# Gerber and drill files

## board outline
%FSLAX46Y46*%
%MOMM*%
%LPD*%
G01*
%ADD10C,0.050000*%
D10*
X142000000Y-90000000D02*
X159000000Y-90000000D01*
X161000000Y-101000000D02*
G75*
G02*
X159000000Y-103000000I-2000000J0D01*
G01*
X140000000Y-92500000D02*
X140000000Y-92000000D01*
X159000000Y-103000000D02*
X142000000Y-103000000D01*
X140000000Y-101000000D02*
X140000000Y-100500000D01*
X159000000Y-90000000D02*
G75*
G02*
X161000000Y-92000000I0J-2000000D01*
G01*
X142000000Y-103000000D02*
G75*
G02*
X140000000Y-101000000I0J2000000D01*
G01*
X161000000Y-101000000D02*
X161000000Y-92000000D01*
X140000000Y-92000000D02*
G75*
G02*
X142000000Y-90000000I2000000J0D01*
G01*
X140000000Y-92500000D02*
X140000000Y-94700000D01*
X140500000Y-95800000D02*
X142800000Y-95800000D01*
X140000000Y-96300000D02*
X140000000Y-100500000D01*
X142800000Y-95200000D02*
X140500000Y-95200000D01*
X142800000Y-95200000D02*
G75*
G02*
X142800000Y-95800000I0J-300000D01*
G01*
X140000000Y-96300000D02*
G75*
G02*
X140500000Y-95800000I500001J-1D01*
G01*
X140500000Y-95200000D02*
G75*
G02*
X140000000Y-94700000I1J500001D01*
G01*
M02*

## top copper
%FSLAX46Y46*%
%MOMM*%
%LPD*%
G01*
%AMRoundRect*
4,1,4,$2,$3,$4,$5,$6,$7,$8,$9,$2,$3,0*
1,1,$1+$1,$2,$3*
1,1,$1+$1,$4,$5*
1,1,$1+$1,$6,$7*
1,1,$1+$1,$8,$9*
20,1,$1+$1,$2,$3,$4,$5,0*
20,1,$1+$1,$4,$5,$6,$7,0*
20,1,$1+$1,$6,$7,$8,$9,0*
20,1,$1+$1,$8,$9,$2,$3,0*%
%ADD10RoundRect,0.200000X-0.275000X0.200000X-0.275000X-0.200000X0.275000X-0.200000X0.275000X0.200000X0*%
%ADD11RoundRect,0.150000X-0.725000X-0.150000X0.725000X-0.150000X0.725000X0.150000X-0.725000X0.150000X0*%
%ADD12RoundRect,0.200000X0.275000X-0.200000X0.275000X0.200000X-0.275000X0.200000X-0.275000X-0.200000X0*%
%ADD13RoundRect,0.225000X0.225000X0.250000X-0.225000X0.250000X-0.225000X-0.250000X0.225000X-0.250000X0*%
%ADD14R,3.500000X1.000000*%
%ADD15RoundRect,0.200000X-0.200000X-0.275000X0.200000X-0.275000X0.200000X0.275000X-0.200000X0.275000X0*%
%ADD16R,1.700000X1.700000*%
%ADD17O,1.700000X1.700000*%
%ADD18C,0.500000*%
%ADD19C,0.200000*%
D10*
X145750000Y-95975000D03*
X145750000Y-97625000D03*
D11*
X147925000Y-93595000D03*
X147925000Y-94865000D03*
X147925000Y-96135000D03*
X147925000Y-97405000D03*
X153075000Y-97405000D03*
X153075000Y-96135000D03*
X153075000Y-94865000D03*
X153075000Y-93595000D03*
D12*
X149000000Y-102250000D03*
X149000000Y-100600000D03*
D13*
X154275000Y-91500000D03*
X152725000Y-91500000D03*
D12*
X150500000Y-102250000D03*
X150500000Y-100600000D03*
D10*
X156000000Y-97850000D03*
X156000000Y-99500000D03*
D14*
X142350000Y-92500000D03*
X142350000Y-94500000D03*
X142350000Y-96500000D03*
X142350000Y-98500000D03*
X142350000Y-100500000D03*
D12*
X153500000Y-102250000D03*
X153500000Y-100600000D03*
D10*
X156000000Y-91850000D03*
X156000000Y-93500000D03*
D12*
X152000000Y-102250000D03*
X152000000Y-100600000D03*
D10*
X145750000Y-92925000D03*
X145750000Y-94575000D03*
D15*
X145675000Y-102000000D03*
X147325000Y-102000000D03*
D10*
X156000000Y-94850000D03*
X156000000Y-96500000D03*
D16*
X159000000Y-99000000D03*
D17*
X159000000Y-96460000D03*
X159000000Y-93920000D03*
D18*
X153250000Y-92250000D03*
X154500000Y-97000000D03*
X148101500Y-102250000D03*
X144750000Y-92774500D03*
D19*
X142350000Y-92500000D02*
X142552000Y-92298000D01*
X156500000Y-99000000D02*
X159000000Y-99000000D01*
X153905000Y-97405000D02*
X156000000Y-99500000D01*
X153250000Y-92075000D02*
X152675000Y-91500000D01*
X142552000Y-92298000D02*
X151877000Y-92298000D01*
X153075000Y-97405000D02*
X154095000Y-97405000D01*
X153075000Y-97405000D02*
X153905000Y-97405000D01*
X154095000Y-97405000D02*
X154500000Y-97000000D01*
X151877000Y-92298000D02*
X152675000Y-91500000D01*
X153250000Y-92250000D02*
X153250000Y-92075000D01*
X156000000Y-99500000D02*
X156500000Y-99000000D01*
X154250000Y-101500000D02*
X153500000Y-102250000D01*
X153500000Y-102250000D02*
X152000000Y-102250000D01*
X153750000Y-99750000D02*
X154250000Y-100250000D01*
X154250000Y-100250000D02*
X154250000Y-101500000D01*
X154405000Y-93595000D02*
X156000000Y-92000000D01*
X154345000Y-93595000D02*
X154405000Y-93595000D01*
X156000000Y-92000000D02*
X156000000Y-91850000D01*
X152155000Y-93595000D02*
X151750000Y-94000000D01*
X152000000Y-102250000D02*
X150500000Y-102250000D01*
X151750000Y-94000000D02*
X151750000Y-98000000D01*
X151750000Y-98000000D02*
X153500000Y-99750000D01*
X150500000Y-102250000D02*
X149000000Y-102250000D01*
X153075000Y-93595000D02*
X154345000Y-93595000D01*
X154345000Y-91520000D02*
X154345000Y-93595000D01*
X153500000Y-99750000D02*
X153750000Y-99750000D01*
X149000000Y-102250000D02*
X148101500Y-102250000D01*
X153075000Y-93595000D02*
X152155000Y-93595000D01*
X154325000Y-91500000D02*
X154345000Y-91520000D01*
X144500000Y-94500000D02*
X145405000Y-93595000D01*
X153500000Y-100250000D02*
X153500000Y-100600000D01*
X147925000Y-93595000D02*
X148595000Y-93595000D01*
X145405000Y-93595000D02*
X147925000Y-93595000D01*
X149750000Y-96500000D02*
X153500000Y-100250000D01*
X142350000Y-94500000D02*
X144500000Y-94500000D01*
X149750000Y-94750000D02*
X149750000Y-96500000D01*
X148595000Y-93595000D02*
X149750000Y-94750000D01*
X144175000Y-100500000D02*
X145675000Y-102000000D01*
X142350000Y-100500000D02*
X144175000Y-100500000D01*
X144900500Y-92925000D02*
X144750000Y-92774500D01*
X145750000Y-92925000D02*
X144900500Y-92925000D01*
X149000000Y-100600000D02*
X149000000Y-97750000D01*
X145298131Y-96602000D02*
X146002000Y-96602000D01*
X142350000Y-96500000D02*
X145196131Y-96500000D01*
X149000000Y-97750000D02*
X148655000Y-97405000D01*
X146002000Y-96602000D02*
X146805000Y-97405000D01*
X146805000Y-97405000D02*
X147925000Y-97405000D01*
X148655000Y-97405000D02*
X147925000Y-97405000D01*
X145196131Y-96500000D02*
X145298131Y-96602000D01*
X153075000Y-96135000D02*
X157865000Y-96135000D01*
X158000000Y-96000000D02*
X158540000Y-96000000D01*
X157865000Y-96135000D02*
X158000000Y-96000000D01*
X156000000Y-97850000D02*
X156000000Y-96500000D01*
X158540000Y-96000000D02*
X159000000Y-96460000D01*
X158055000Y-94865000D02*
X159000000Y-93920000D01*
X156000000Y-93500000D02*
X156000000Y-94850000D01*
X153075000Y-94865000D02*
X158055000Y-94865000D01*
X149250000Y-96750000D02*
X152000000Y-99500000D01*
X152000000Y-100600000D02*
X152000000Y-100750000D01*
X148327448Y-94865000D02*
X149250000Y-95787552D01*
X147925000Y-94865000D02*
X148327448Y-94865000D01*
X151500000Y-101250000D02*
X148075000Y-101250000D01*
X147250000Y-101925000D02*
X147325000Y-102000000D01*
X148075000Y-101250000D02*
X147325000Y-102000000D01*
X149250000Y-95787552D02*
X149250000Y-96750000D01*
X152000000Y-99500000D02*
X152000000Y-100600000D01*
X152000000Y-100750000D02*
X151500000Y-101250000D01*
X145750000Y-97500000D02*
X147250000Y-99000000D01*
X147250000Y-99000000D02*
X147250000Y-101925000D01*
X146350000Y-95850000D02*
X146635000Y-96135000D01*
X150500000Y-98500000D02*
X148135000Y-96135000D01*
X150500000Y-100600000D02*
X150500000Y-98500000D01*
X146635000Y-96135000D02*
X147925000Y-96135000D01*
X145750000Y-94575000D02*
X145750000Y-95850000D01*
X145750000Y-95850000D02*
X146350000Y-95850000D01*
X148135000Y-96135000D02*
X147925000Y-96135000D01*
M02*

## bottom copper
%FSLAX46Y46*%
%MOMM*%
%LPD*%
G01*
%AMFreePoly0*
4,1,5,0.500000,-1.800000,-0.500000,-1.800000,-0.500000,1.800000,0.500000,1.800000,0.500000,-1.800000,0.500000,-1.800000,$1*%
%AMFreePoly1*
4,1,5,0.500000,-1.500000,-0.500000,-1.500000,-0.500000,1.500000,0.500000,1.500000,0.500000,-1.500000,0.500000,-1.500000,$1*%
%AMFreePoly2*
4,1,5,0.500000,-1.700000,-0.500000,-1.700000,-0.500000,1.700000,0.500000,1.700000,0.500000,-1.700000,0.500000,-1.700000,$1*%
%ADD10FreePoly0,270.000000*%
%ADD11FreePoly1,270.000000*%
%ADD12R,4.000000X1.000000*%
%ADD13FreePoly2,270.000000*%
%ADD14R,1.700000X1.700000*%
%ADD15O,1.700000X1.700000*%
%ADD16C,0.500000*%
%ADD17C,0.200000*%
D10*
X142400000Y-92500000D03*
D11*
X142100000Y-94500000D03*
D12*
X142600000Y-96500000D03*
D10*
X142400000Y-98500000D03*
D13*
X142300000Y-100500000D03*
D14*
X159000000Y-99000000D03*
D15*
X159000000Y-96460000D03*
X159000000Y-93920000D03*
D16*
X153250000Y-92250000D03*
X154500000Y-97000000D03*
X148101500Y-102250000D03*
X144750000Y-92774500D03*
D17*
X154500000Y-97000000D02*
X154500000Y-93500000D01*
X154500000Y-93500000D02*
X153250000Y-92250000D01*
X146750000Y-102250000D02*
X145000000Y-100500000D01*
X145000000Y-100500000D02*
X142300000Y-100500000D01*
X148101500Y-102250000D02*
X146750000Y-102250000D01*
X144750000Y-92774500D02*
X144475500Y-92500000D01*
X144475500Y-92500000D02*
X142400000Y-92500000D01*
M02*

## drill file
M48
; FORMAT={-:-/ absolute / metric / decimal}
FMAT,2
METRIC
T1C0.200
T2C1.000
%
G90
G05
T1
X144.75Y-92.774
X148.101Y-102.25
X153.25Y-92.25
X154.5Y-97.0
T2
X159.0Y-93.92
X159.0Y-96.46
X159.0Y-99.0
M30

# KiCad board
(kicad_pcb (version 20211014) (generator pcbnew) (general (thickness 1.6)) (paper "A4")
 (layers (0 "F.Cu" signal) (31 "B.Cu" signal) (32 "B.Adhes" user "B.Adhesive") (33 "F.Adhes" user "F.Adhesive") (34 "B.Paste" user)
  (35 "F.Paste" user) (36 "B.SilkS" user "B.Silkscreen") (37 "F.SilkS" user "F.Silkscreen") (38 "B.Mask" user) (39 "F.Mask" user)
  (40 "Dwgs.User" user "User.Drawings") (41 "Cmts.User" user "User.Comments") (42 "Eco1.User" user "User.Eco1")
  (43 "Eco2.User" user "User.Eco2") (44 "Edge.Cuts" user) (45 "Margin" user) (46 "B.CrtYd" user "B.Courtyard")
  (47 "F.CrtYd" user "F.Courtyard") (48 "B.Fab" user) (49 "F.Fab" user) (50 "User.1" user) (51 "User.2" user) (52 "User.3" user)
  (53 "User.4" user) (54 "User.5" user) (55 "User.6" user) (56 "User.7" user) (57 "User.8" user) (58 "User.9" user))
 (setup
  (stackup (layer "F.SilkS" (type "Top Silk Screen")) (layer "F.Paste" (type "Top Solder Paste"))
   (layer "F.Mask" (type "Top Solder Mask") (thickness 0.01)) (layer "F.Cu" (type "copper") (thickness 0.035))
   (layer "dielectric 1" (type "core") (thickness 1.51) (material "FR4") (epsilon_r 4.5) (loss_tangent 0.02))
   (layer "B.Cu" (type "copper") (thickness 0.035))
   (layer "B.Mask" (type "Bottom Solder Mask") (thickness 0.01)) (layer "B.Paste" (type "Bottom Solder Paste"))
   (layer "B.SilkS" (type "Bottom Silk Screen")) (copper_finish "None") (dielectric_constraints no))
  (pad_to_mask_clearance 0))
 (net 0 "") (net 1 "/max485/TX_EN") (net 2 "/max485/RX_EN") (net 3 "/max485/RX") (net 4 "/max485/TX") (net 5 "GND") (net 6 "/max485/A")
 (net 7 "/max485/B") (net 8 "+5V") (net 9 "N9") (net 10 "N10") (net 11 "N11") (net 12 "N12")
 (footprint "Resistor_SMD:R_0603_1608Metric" (layer "F.Cu") (at 145.75 96.8 -90)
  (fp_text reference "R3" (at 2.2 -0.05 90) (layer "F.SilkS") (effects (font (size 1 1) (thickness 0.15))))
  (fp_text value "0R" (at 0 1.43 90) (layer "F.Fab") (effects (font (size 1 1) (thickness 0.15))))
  (pad "1" smd roundrect (at -0.825 0 270) (size 0.8 0.95) (layers "F.Cu" "F.Paste" "F.Mask") (roundrect_rratio 0.25)
   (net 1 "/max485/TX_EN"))
  (pad "2" smd roundrect (at 0.825 0 270) (size 0.8 0.95) (layers "F.Cu" "F.Paste" "F.Mask") (roundrect_rratio 0.25) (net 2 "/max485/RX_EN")))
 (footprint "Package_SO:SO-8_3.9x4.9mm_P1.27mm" (layer "F.Cu") (at 150.5 95.5)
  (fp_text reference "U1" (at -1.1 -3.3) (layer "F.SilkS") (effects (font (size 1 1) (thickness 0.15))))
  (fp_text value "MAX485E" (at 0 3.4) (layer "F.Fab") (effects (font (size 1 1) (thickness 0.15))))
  (pad "1" smd roundrect (at -2.575 -1.905) (size 1.75 0.6) (layers "F.Cu" "F.Paste" "F.Mask") (roundrect_rratio 0.25) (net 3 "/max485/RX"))
  (pad "2" smd roundrect (at -2.575 -0.635) (size 1.75 0.6) (layers "F.Cu" "F.Paste" "F.Mask") (roundrect_rratio 0.25)
   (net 2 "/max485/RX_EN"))
  (pad "3" smd roundrect (at -2.575 0.635) (size 1.75 0.6) (layers "F.Cu" "F.Paste" "F.Mask") (roundrect_rratio 0.25)
   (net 1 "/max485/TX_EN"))
  (pad "4" smd roundrect (at -2.575 1.905) (size 1.75 0.6) (layers "F.Cu" "F.Paste" "F.Mask") (roundrect_rratio 0.25) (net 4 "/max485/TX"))
  (pad "5" smd roundrect (at 2.575 1.905) (size 1.75 0.6) (layers "F.Cu" "F.Paste" "F.Mask") (roundrect_rratio 0.25) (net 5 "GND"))
  (pad "6" smd roundrect (at 2.575 0.635) (size 1.75 0.6) (layers "F.Cu" "F.Paste" "F.Mask") (roundrect_rratio 0.25) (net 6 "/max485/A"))
  (pad "7" smd roundrect (at 2.575 -0.635) (size 1.75 0.6) (layers "F.Cu" "F.Paste" "F.Mask") (roundrect_rratio 0.25) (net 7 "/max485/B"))
  (pad "8" smd roundrect (at 2.575 -1.905) (size 1.75 0.6) (layers "F.Cu" "F.Paste" "F.Mask") (roundrect_rratio 0.25) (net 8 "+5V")))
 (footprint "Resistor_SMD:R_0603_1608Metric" (layer "F.Cu") (at 149 101.425 90)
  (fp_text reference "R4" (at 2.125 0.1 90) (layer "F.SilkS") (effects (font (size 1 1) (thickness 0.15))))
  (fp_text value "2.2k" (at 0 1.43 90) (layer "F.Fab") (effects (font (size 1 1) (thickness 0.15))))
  (pad "1" smd roundrect (at -0.825 0 90) (size 0.8 0.95) (layers "F.Cu" "F.Paste" "F.Mask") (roundrect_rratio 0.25) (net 8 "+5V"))
  (pad "2" smd roundrect (at 0.825 0 90) (size 0.8 0.95) (layers "F.Cu" "F.Paste" "F.Mask") (roundrect_rratio 0.25) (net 4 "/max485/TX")))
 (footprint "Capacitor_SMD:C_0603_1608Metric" (layer "F.Cu") (at 153.5 91.5 180)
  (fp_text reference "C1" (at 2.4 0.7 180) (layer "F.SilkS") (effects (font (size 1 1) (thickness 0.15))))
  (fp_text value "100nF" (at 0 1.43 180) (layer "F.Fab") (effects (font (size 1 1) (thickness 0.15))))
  (pad "1" smd roundrect (at -0.775 0 180) (size 0.9 0.95) (layers "F.Cu" "F.Paste" "F.Mask") (roundrect_rratio 0.25) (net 8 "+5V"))
  (pad "2" smd roundrect (at 0.775 0 180) (size 0.9 0.95) (layers "F.Cu" "F.Paste" "F.Mask") (roundrect_rratio 0.25) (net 5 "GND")))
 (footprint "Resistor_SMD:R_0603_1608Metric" (layer "F.Cu") (at 150.5 101.425 90)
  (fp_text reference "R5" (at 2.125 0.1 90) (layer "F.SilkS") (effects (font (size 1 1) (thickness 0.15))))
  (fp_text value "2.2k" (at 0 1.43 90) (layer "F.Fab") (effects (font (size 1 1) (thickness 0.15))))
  (pad "1" smd roundrect (at -0.825 0 90) (size 0.8 0.95) (layers "F.Cu" "F.Paste" "F.Mask") (roundrect_rratio 0.25) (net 8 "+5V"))
  (pad "2" smd roundrect (at 0.825 0 90) (size 0.8 0.95) (layers "F.Cu" "F.Paste" "F.Mask") (roundrect_rratio 0.25) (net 1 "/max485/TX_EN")))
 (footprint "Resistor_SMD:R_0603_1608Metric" (layer "F.Cu") (at 156 98.675 -90)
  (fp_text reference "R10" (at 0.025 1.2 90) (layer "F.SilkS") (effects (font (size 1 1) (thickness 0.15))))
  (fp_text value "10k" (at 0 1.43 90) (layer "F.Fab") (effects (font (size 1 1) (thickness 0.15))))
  (pad "1" smd roundrect (at -0.825 0 270) (size 0.8 0.95) (layers "F.Cu" "F.Paste" "F.Mask") (roundrect_rratio 0.25) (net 6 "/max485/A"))
  (pad "2" smd roundrect (at 0.825 0 270) (size 0.8 0.95) (layers "F.Cu" "F.Paste" "F.Mask") (roundrect_rratio 0.25) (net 5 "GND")))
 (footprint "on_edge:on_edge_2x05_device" (layer "F.Cu") (at 140 96.5 -90)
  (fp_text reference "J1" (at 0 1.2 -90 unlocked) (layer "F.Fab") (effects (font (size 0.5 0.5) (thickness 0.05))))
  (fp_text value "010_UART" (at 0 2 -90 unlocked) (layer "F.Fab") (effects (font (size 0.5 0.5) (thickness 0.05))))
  (fp_line (start -4 0) (end -1.8 0) (layer "Edge.Cuts") (width 0.05))
  (fp_line (start -0.7 -0.5) (end -0.7 -2.8) (layer "Edge.Cuts") (width 0.05))
  (fp_line (start -0.2 0) (end 4 0) (layer "Edge.Cuts") (width 0.05))
  (fp_line (start -1.3 -2.8) (end -1.3 -0.5) (layer "Edge.Cuts") (width 0.05))
  (fp_arc (start -1.3 -2.8) (mid -1 -3.1) (end -0.7 -2.8) (layer "Edge.Cuts") (width 0.05))
  (fp_arc (start -0.2 0) (mid -0.553553 -0.146447) (end -0.7 -0.5) (layer "Edge.Cuts") (width 0.05))
  (fp_arc (start -1.3 -0.5) (mid -1.446447 -0.146447) (end -1.8 0) (layer "Edge.Cuts") (width 0.05))
  (pad "1" smd rect (at -4 -2.35 90) (size 1 3.5) (layers "F.Cu" "F.Mask") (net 5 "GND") (zone_connect 0))
  (pad "2" smd rect (at -2 -2.35 270) (size 1 3.5) (layers "F.Cu" "F.Mask") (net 3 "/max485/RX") (zone_connect 0))
  (pad "3" smd rect (at 0 -2.35 270) (size 1 3.5) (layers "F.Cu" "F.Mask") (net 4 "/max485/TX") (zone_connect 0))
  (pad "4" smd rect (at 2 -2.35 90) (size 1 3.5) (layers "F.Cu" "F.Mask") (zone_connect 0))
  (pad "5" smd rect (at 4 -2.35 90) (size 1 3.5) (layers "F.Cu" "F.Mask") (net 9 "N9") (zone_connect 0))
  (pad "6" smd custom (at -4 -2.4 270) (size 1 3.6) (layers "B.Cu" "B.Mask") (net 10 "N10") (zone_connect 0)
   (options (clearance outline) (anchor rect)) (primitives))
  (pad "7" smd custom (at -2 -2.1 270) (size 1 3) (layers "B.Cu" "B.Mask") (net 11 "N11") (zone_connect 0)
   (options (clearance outline) (anchor rect)) (primitives))
  (pad "8" smd rect (at 0 -2.6 270) (size 1 4) (layers "B.Cu" "B.Mask") (zone_connect 0))
  (pad "9" smd custom (at 2 -2.4 270) (size 1 3.6) (layers "B.Cu" "B.Mask") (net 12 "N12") (zone_connect 0)
   (options (clearance outline) (anchor rect)) (primitives))
  (pad "10" smd custom (at 4 -2.3 270) (size 1 3.4) (layers "B.Cu" "B.Mask") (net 8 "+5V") (zone_connect 0)
   (options (clearance outline) (anchor rect)) (primitives)))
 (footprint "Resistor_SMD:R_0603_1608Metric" (layer "F.Cu") (at 153.5 101.425 90)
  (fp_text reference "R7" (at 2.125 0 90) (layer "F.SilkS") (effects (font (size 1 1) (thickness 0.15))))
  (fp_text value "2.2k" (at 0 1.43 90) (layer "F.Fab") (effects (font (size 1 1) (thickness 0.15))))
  (pad "1" smd roundrect (at -0.825 0 90) (size 0.8 0.95) (layers "F.Cu" "F.Paste" "F.Mask") (roundrect_rratio 0.25) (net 8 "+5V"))
  (pad "2" smd roundrect (at 0.825 0 90) (size 0.8 0.95) (layers "F.Cu" "F.Paste" "F.Mask") (roundrect_rratio 0.25) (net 3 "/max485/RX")))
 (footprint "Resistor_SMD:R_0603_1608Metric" (layer "F.Cu") (at 156 92.675 -90)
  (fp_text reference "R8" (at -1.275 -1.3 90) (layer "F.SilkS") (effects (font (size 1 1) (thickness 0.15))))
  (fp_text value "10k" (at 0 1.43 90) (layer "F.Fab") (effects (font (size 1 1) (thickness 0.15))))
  (pad "1" smd roundrect (at -0.825 0 270) (size 0.8 0.95) (layers "F.Cu" "F.Paste" "F.Mask") (roundrect_rratio 0.25) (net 8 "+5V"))
  (pad "2" smd roundrect (at 0.825 0 270) (size 0.8 0.95) (layers "F.Cu" "F.Paste" "F.Mask") (roundrect_rratio 0.25) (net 7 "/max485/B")))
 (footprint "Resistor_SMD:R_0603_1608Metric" (layer "F.Cu") (at 152 101.425 90)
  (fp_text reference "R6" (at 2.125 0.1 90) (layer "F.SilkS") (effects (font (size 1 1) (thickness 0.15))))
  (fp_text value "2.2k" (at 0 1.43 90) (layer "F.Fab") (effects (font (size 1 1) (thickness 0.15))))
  (pad "1" smd roundrect (at -0.825 0 90) (size 0.8 0.95) (layers "F.Cu" "F.Paste" "F.Mask") (roundrect_rratio 0.25) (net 8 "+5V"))
  (pad "2" smd roundrect (at 0.825 0 90) (size 0.8 0.95) (layers "F.Cu" "F.Paste" "F.Mask") (roundrect_rratio 0.25) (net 2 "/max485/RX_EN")))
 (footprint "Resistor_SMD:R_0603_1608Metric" (layer "F.Cu") (at 145.75 93.75 -90)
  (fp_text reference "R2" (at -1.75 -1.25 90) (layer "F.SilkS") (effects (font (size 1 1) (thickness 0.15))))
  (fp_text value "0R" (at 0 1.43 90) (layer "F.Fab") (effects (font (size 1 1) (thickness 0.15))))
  (pad "1" smd roundrect (at -0.825 0 270) (size 0.8 0.95) (layers "F.Cu" "F.Paste" "F.Mask") (roundrect_rratio 0.25) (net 10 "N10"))
  (pad "2" smd roundrect (at 0.825 0 270) (size 0.8 0.95) (layers "F.Cu" "F.Paste" "F.Mask") (roundrect_rratio 0.25) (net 1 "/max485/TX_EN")))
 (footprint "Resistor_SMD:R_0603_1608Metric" (layer "F.Cu") (at 146.5 102)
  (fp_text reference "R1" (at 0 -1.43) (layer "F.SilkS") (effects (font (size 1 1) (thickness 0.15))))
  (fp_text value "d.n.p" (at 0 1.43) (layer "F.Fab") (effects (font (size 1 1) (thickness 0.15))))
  (pad "1" smd roundrect (at -0.825 0) (size 0.8 0.95) (layers "F.Cu" "F.Paste" "F.Mask") (roundrect_rratio 0.25) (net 9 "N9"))
  (pad "2" smd roundrect (at 0.825 0) (size 0.8 0.95) (layers "F.Cu" "F.Paste" "F.Mask") (roundrect_rratio 0.25) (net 2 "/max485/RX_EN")))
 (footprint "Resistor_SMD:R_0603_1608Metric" (layer "F.Cu") (at 156 95.675 -90)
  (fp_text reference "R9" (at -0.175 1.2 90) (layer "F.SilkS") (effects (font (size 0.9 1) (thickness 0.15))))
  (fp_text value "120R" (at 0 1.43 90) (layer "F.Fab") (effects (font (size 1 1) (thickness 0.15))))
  (pad "1" smd roundrect (at -0.825 0 270) (size 0.8 0.95) (layers "F.Cu" "F.Paste" "F.Mask") (roundrect_rratio 0.25) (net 7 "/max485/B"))
  (pad "2" smd roundrect (at 0.825 0 270) (size 0.8 0.95) (layers "F.Cu" "F.Paste" "F.Mask") (roundrect_rratio 0.25) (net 6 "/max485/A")))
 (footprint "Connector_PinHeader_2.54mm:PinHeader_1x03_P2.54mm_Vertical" (layer "F.Cu") (at 159 99 180)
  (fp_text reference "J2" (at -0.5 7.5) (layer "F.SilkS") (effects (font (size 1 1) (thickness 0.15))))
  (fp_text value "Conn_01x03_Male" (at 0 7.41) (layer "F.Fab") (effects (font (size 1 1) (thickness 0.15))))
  (pad "1" thru_hole rect (at 0 0 180) (size 1.7 1.7) (drill 1) (layers *.Cu *.Mask) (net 5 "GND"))
  (pad "2" thru_hole oval (at 0 2.54 180) (size 1.7 1.7) (drill 1) (layers *.Cu *.Mask) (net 6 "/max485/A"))
  (pad "3" thru_hole oval (at 0 5.08 180) (size 1.7 1.7) (drill 1) (layers *.Cu *.Mask) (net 7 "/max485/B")))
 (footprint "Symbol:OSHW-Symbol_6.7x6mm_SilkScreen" (layer "B.Cu") (at 151 96.5 180)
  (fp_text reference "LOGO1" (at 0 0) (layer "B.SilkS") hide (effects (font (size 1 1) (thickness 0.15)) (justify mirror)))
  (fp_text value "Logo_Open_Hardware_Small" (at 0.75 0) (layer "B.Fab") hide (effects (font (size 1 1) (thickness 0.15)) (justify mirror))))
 (gr_line (start 142 90) (end 159 90) (layer "Edge.Cuts") (width 0.05))
 (gr_arc (start 161 101) (mid 160.414214 102.414214) (end 159 103) (layer "Edge.Cuts") (width 0.05))
 (gr_line (start 140 92.5) (end 140 92) (layer "Edge.Cuts") (width 0.05))
 (gr_line (start 159 103) (end 142 103) (layer "Edge.Cuts") (width 0.05))
 (gr_line (start 140 101) (end 140 100.5) (layer "Edge.Cuts") (width 0.05))
 (gr_arc (start 159 90) (mid 160.414214 90.585786) (end 161 92) (layer "Edge.Cuts") (width 0.05))
 (gr_arc (start 142 103) (mid 140.585786 102.414214) (end 140 101) (layer "Edge.Cuts") (width 0.05))
 (gr_line (start 161 101) (end 161 92) (layer "Edge.Cuts") (width 0.05))
 (gr_arc (start 140 92) (mid 140.585786 90.585786) (end 142 90) (layer "Edge.Cuts") (width 0.05))
 (segment (start 142.35 92.5) (end 142.552 92.298) (width 0.2) (layer "F.Cu") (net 5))
 (segment (start 156.5 99) (end 159 99) (width 0.2) (layer "F.Cu") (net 5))
 (segment (start 153.905 97.405) (end 156 99.5) (width 0.2) (layer "F.Cu") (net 5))
 (segment (start 153.25 92.075) (end 152.675 91.5) (width 0.2) (layer "F.Cu") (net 5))
 (segment (start 142.552 92.298) (end 151.877 92.298) (width 0.2) (layer "F.Cu") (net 5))
 (segment (start 153.075 97.405) (end 154.095 97.405) (width 0.2) (layer "F.Cu") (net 5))
 (segment (start 153.075 97.405) (end 153.905 97.405) (width 0.2) (layer "F.Cu") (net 5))
 (segment (start 154.095 97.405) (end 154.5 97) (width 0.2) (layer "F.Cu") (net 5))
 (segment (start 151.877 92.298) (end 152.675 91.5) (width 0.2) (layer "F.Cu") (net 5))
 (segment (start 153.25 92.25) (end 153.25 92.075) (width 0.2) (layer "F.Cu") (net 5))
 (segment (start 156 99.5) (end 156.5 99) (width 0.2) (layer "F.Cu") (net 5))
 (via (at 153.25 92.25) (size 0.5) (drill 0.2) (layers "F.Cu" "B.Cu") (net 5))
 (via (at 154.5 97) (size 0.5) (drill 0.2) (layers "F.Cu" "B.Cu") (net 5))
 (segment (start 154.5 97) (end 154.5 93.5) (width 0.2) (layer "B.Cu") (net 5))
 (segment (start 154.5 93.5) (end 153.25 92.25) (width 0.2) (layer "B.Cu") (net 5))
 (segment (start 154.25 101.5) (end 153.5 102.25) (width 0.2) (layer "F.Cu") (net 8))
 (segment (start 153.5 102.25) (end 152 102.25) (width 0.2) (layer "F.Cu") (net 8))
 (segment (start 153.75 99.75) (end 154.25 100.25) (width 0.2) (layer "F.Cu") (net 8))
 (segment (start 154.25 100.25) (end 154.25 101.5) (width 0.2) (layer "F.Cu") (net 8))
 (segment (start 154.405 93.595) (end 156 92) (width 0.2) (layer "F.Cu") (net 8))
 (segment (start 154.345 93.595) (end 154.405 93.595) (width 0.2) (layer "F.Cu") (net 8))
 (segment (start 156 92) (end 156 91.85) (width 0.2) (layer "F.Cu") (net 8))
 (segment (start 152.155 93.595) (end 151.75 94) (width 0.2) (layer "F.Cu") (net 8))
 (segment (start 152 102.25) (end 150.5 102.25) (width 0.2) (layer "F.Cu") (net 8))
 (segment (start 151.75 94) (end 151.75 98) (width 0.2) (layer "F.Cu") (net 8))
 (segment (start 151.75 98) (end 153.5 99.75) (width 0.2) (layer "F.Cu") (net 8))
 (segment (start 150.5 102.25) (end 149 102.25) (width 0.2) (layer "F.Cu") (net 8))
 (segment (start 153.075 93.595) (end 154.345 93.595) (width 0.2) (layer "F.Cu") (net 8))
 (segment (start 154.345 91.52) (end 154.345 93.595) (width 0.2) (layer "F.Cu") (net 8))
 (segment (start 153.5 99.75) (end 153.75 99.75) (width 0.2) (layer "F.Cu") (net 8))
 (segment (start 149 102.25) (end 148.1015 102.25) (width 0.2) (layer "F.Cu") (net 8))
 (segment (start 153.075 93.595) (end 152.155 93.595) (width 0.2) (layer "F.Cu") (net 8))
 (segment (start 154.325 91.5) (end 154.345 91.52) (width 0.2) (layer "F.Cu") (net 8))
 (via (at 148.1015 102.25) (size 0.5) (drill 0.2) (layers "F.Cu" "B.Cu") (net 8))
 (segment (start 146.75 102.25) (end 145 100.5) (width 0.2) (layer "B.Cu") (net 8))
 (segment (start 145 100.5) (end 142.3 100.5) (width 0.2) (layer "B.Cu") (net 8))
 (segment (start 148.1015 102.25) (end 146.75 102.25) (width 0.2) (layer "B.Cu") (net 8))
 (segment (start 144.5 94.5) (end 145.405 93.595) (width 0.2) (layer "F.Cu") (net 3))
 (segment (start 153.5 100.25) (end 153.5 100.6) (width 0.2) (layer "F.Cu") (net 3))
 (segment (start 147.925 93.595) (end 148.595 93.595) (width 0.2) (layer "F.Cu") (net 3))
 (segment (start 145.405 93.595) (end 147.925 93.595) (width 0.2) (layer "F.Cu") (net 3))
 (segment (start 149.75 96.5) (end 153.5 100.25) (width 0.2) (layer "F.Cu") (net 3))
 (segment (start 142.35 94.5) (end 144.5 94.5) (width 0.2) (layer "F.Cu") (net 3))
 (segment (start 149.75 94.75) (end 149.75 96.5) (width 0.2) (layer "F.Cu") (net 3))
 (segment (start 148.595 93.595) (end 149.75 94.75) (width 0.2) (layer "F.Cu") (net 3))
 (segment (start 144.175 100.5) (end 145.675 102) (width 0.2) (layer "F.Cu") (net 9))
 (segment (start 142.35 100.5) (end 144.175 100.5) (width 0.2) (layer "F.Cu") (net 9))
 (segment (start 144.9005 92.925) (end 144.75 92.7745) (width 0.2) (layer "F.Cu") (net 10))
 (segment (start 145.75 92.925) (end 144.9005 92.925) (width 0.2) (layer "F.Cu") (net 10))
 (via (at 144.75 92.7745) (size 0.5) (drill 0.2) (layers "F.Cu" "B.Cu") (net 10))
 (segment (start 144.75 92.7745) (end 144.4755 92.5) (width 0.2) (layer "B.Cu") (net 10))
 (segment (start 144.4755 92.5) (end 142.4 92.5) (width 0.2) (layer "B.Cu") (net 10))
 (segment (start 149 100.6) (end 149 97.75) (width 0.2) (layer "F.Cu") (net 4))
 (segment (start 145.298131 96.602) (end 146.002 96.602) (width 0.2) (layer "F.Cu") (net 4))
 (segment (start 142.35 96.5) (end 145.196131 96.5) (width 0.2) (layer "F.Cu") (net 4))
 (segment (start 149 97.75) (end 148.655 97.405) (width 0.2) (layer "F.Cu") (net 4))
 (segment (start 146.002 96.602) (end 146.805 97.405) (width 0.2) (layer "F.Cu") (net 4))
 (segment (start 146.805 97.405) (end 147.925 97.405) (width 0.2) (layer "F.Cu") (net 4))
 (segment (start 148.655 97.405) (end 147.925 97.405) (width 0.2) (layer "F.Cu") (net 4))
 (segment (start 145.196131 96.5) (end 145.298131 96.602) (width 0.2) (layer "F.Cu") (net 4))
 (segment (start 153.075 96.135) (end 157.865 96.135) (width 0.2) (layer "F.Cu") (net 6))
 (segment (start 158 96) (end 158.54 96) (width 0.2) (layer "F.Cu") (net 6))
 (segment (start 157.865 96.135) (end 158 96) (width 0.2) (layer "F.Cu") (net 6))
 (segment (start 156 97.85) (end 156 96.5) (width 0.2) (layer "F.Cu") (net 6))
 (segment (start 158.54 96) (end 159 96.46) (width 0.2) (layer "F.Cu") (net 6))
 (segment (start 158.055 94.865) (end 159 93.92) (width 0.2) (layer "F.Cu") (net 7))
 (segment (start 156 93.5) (end 156 94.85) (width 0.2) (layer "F.Cu") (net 7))
 (segment (start 153.075 94.865) (end 158.055 94.865) (width 0.2) (layer "F.Cu") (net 7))
 (segment (start 149.25 96.75) (end 152 99.5) (width 0.2) (layer "F.Cu") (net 2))
 (segment (start 152 100.6) (end 152 100.75) (width 0.2) (layer "F.Cu") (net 2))
 (segment (start 148.327448 94.865) (end 149.25 95.787552) (width 0.2) (layer "F.Cu") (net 2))
 (segment (start 147.925 94.865) (end 148.327448 94.865) (width 0.2) (layer "F.Cu") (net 2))
 (segment (start 151.5 101.25) (end 148.075 101.25) (width 0.2) (layer "F.Cu") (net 2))
 (segment (start 147.25 101.925) (end 147.325 102) (width 0.2) (layer "F.Cu") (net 2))
 (segment (start 148.075 101.25) (end 147.325 102) (width 0.2) (layer "F.Cu") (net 2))
 (segment (start 149.25 95.787552) (end 149.25 96.75) (width 0.2) (layer "F.Cu") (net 2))
 (segment (start 152 99.5) (end 152 100.6) (width 0.2) (layer "F.Cu") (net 2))
 (segment (start 152 100.75) (end 151.5 101.25) (width 0.2) (layer "F.Cu") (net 2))
 (segment (start 145.75 97.5) (end 147.25 99) (width 0.2) (layer "F.Cu") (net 2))
 (segment (start 147.25 99) (end 147.25 101.925) (width 0.2) (layer "F.Cu") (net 2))
 (segment (start 146.35 95.85) (end 146.635 96.135) (width 0.2) (layer "F.Cu") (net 1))
 (segment (start 150.5 98.5) (end 148.135 96.135) (width 0.2) (layer "F.Cu") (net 1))
 (segment (start 150.5 100.6) (end 150.5 98.5) (width 0.2) (layer "F.Cu") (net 1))
 (segment (start 146.635 96.135) (end 147.925 96.135) (width 0.2) (layer "F.Cu") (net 1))
 (segment (start 145.75 94.575) (end 145.75 95.85) (width 0.2) (layer "F.Cu") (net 1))
 (segment (start 145.75 95.85) (end 146.35 95.85) (width 0.2) (layer "F.Cu") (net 1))
 (segment (start 148.135 96.135) (end 147.925 96.135) (width 0.2) (layer "F.Cu") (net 1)))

